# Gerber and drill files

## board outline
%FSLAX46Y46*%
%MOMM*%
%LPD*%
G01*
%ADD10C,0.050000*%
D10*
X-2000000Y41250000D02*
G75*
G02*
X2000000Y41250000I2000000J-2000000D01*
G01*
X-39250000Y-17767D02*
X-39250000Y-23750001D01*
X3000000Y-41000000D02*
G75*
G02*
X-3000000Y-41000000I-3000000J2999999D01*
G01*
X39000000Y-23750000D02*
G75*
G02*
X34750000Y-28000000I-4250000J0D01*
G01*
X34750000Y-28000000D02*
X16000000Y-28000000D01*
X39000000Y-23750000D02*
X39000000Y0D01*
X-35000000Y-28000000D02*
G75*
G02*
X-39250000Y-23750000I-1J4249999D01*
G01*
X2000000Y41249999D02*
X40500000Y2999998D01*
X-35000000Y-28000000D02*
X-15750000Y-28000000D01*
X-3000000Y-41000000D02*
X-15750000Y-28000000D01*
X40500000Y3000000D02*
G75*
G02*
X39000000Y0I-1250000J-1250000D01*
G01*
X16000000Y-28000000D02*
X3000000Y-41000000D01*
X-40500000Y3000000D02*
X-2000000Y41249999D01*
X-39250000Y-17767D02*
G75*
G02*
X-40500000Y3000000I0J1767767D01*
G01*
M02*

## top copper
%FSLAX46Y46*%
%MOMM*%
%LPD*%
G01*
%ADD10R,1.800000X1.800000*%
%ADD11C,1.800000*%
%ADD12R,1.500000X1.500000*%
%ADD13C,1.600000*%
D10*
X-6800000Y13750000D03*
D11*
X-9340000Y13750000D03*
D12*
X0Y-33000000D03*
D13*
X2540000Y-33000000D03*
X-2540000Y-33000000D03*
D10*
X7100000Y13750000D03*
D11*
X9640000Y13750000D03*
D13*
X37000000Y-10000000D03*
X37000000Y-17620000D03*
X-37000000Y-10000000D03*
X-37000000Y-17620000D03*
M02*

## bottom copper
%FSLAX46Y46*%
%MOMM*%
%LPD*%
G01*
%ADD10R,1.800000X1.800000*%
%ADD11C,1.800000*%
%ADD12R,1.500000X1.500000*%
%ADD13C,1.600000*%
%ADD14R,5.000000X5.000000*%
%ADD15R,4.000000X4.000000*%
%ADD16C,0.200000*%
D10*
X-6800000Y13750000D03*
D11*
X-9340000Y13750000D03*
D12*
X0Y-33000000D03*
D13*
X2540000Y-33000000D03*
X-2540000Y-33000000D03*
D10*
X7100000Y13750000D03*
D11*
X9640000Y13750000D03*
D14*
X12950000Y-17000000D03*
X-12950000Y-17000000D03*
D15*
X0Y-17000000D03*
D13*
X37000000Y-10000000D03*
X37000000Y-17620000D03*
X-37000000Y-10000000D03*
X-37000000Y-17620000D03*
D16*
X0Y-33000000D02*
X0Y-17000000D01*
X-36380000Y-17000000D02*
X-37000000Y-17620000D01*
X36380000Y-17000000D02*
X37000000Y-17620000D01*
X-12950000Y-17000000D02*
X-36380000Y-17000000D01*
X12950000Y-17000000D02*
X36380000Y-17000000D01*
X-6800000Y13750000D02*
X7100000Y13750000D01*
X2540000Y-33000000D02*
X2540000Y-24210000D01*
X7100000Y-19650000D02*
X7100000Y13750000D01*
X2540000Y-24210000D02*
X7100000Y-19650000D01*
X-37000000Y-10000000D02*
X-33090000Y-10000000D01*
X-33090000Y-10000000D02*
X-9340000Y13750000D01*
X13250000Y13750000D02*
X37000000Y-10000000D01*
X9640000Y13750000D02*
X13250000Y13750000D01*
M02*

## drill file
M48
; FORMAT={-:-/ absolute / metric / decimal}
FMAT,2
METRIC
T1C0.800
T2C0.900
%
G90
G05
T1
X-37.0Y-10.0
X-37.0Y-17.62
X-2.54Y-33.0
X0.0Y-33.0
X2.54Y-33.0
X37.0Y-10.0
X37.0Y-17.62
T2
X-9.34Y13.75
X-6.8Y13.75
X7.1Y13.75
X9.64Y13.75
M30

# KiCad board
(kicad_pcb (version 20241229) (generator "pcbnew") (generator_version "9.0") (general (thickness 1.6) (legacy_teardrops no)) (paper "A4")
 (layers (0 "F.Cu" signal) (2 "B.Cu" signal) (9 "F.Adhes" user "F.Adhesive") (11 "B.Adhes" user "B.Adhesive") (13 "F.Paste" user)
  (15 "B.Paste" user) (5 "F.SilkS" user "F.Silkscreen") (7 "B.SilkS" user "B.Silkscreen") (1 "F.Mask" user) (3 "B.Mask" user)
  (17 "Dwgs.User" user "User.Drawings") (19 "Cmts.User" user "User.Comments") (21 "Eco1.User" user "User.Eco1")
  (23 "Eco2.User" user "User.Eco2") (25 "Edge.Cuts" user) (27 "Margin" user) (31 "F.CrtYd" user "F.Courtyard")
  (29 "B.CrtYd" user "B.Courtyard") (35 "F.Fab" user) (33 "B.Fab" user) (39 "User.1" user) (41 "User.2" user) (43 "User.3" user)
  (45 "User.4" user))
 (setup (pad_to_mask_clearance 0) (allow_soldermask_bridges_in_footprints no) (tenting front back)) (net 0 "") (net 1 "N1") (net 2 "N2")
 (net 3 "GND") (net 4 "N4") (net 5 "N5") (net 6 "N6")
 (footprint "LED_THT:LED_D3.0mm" (layer "F.Cu") (at -6.8 -13.75 180)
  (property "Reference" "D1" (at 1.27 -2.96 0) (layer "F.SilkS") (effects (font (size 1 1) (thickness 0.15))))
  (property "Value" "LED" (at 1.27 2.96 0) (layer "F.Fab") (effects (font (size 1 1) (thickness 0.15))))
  (pad "1" thru_hole rect (at 0 0 180) (size 1.8 1.8) (drill 0.9) (layers "*.Cu" "*.Mask") (remove_unused_layers no) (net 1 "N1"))
  (pad "2" thru_hole circle (at 2.54 0 180) (size 1.8 1.8) (drill 0.9) (layers "*.Cu" "*.Mask") (remove_unused_layers no) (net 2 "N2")))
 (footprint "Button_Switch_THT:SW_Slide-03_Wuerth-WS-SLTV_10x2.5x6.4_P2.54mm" (layer "F.Cu") (at 0 33 180)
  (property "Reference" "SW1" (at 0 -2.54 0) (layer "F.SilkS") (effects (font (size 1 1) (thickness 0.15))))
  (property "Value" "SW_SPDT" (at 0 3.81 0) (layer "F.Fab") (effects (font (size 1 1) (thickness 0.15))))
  (pad "1" thru_hole rect (at 0 0 180) (size 1.5 1.5) (drill 0.8) (layers "*.Cu" "*.Mask") (remove_unused_layers no) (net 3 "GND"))
  (pad "2" thru_hole circle (at -2.54 0 180) (size 1.6 1.6) (drill 0.8) (layers "*.Cu" "*.Mask") (remove_unused_layers no) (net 1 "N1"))
  (pad "3" thru_hole circle (at 2.54 0 180) (size 1.6 1.6) (drill 0.8) (layers "*.Cu" "*.Mask") (remove_unused_layers no) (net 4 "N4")))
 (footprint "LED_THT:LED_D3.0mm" (layer "F.Cu") (at 7.1 -13.75)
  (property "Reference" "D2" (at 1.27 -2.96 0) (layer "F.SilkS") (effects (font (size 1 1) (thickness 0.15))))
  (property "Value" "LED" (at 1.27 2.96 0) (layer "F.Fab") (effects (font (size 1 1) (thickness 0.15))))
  (pad "1" thru_hole rect (at 0 0) (size 1.8 1.8) (drill 0.9) (layers "*.Cu" "*.Mask") (remove_unused_layers no) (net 1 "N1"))
  (pad "2" thru_hole circle (at 2.54 0) (size 1.8 1.8) (drill 0.9) (layers "*.Cu" "*.Mask") (remove_unused_layers no) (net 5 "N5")))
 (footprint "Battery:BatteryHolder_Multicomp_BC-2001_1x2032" (layer "B.Cu") (at 0 17 180)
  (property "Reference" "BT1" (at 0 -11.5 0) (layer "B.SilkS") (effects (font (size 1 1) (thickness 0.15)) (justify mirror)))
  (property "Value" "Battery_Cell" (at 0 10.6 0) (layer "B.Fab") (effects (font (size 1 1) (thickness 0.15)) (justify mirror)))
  (pad "1" smd rect (at -12.95 0 180) (size 5 5) (layers "B.Cu" "B.Mask" "B.Paste") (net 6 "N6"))
  (pad "1" smd rect (at 12.95 0 180) (size 5 5) (layers "B.Cu" "B.Mask" "B.Paste") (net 6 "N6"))
  (pad "2" smd rect (at 0 0 180) (size 4 4) (layers "B.Cu" "B.Mask" "B.Paste") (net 3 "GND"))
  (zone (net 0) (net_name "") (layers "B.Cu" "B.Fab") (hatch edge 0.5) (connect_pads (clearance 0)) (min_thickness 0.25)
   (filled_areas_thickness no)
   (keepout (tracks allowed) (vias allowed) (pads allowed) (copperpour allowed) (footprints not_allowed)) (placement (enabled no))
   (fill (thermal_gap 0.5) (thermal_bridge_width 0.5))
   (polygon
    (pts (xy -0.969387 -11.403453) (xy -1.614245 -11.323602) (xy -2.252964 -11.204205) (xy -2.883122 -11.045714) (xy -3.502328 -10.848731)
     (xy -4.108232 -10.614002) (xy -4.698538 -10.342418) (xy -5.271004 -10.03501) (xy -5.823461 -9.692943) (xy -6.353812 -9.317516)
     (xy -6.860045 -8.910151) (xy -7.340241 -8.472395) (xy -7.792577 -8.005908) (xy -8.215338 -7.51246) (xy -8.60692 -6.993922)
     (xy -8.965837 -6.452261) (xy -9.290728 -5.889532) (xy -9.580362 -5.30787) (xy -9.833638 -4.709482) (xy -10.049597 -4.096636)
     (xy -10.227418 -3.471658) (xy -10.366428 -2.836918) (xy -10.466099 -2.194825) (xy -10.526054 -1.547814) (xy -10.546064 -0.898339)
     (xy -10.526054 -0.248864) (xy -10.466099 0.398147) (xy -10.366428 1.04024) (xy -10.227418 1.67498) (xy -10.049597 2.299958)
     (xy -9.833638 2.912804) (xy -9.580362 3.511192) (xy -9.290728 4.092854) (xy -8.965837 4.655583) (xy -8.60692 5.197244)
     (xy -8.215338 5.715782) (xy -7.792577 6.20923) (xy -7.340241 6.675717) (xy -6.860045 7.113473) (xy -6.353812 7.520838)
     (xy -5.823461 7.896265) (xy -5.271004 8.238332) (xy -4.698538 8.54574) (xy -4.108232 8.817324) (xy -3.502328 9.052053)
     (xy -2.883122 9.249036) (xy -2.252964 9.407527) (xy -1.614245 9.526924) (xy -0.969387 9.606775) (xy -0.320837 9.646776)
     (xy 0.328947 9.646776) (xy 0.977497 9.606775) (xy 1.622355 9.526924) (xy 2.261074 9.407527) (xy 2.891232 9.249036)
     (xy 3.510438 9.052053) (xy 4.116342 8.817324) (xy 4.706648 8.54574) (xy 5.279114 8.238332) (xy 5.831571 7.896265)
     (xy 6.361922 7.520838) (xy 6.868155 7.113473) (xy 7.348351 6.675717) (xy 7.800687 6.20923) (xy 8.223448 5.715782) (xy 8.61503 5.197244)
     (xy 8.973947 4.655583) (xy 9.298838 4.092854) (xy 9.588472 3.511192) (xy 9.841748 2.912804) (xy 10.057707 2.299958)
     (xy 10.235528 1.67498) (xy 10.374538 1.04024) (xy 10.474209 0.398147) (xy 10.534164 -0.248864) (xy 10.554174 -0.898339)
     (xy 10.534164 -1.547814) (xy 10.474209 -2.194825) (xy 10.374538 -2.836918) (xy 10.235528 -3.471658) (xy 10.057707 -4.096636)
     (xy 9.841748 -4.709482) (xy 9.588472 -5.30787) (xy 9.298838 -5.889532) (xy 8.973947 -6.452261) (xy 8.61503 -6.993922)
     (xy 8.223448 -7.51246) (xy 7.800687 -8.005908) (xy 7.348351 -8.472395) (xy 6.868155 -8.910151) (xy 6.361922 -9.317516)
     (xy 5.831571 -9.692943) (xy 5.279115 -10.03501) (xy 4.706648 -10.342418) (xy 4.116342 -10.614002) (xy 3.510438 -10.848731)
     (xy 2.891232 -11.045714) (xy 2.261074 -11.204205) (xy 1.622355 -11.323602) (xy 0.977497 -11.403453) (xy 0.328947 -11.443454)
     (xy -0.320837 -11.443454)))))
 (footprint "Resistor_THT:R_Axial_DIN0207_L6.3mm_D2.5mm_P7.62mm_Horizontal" (layer "B.Cu") (at 37 10 -90)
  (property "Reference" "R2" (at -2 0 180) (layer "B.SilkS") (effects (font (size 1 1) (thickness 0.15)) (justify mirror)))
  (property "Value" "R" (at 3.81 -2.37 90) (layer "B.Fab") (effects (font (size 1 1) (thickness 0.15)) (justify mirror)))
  (pad "1" thru_hole circle (at 0 0 270) (size 1.6 1.6) (drill 0.8) (layers "*.Cu" "*.Mask") (remove_unused_layers no) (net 5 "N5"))
  (pad "2" thru_hole circle (at 7.62 0 270) (size 1.6 1.6) (drill 0.8) (layers "*.Cu" "*.Mask") (remove_unused_layers no) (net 6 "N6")))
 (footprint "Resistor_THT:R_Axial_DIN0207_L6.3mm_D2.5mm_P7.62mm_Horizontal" (layer "B.Cu") (at -37 10 -90)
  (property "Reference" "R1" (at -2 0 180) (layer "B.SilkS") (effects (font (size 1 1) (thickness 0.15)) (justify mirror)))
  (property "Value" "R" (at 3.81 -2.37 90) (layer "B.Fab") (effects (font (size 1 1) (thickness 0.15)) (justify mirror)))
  (pad "1" thru_hole circle (at 0 0 270) (size 1.6 1.6) (drill 0.8) (layers "*.Cu" "*.Mask") (remove_unused_layers no) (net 2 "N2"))
  (pad "2" thru_hole circle (at 7.62 0 270) (size 1.6 1.6) (drill 0.8) (layers "*.Cu" "*.Mask") (remove_unused_layers no) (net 6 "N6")))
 (gr_arc (start -2 -41.25) (mid 0 -42.078427) (end 2 -41.25) (stroke (width 0.05) (type default)) (layer "Edge.Cuts"))
 (gr_line (start -39.25 0.017767) (end -39.25 23.750001) (stroke (width 0.05) (type default)) (layer "Edge.Cuts"))
 (gr_arc (start 3 41) (mid 0 42.242641) (end -3 41) (stroke (width 0.05) (type default)) (layer "Edge.Cuts"))
 (gr_arc (start 39 23.75) (mid 37.755204 26.755204) (end 34.75 28) (stroke (width 0.05) (type default)) (layer "Edge.Cuts"))
 (gr_line (start 34.75 28) (end 16 28) (stroke (width 0.05) (type default)) (layer "Edge.Cuts"))
 (gr_line (start 39 23.75) (end 39 0) (stroke (width 0.05) (type default)) (layer "Edge.Cuts"))
 (gr_arc (start -35 28) (mid -38.005204 26.755204) (end -39.25 23.75) (stroke (width 0.05) (type default)) (layer "Edge.Cuts"))
 (gr_line (start 2 -41.249999) (end 40.5 -2.999998) (stroke (width 0.05) (type default)) (layer "Edge.Cuts"))
 (gr_line (start -35 28) (end -15.75 28) (stroke (width 0.05) (type default)) (layer "Edge.Cuts"))
 (gr_line (start -3 41) (end -15.75 28) (stroke (width 0.05) (type default)) (layer "Edge.Cuts"))
 (gr_arc (start 40.5 -3) (mid 40.831139 -0.959431) (end 39 0) (stroke (width 0.05) (type default)) (layer "Edge.Cuts"))
 (gr_line (start 16 28) (end 3 41) (stroke (width 0.05) (type default)) (layer "Edge.Cuts"))
 (gr_line (start -40.5 -3) (end -2 -41.249999) (stroke (width 0.05) (type default)) (layer "Edge.Cuts"))
 (gr_arc (start -39.25 0.017767) (mid -40.883204 -1.073505) (end -40.5 -3) (stroke (width 0.05) (type default)) (layer "Edge.Cuts"))
 (segment (start 0 33) (end 0 17) (width 0.2) (layer "B.Cu") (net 3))
 (segment (start -36.38 17) (end -37 17.62) (width 0.2) (layer "B.Cu") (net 6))
 (segment (start 36.38 17) (end 37 17.62) (width 0.2) (layer "B.Cu") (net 6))
 (segment (start -12.95 17) (end -36.38 17) (width 0.2) (layer "B.Cu") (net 6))
 (segment (start 12.95 17) (end 36.38 17) (width 0.2) (layer "B.Cu") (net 6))
 (segment (start -6.8 -13.75) (end 7.1 -13.75) (width 0.2) (layer "B.Cu") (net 1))
 (segment (start 2.54 33) (end 2.54 24.21) (width 0.2) (layer "B.Cu") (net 1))
 (segment (start 7.1 19.65) (end 7.1 -13.75) (width 0.2) (layer "B.Cu") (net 1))
 (segment (start 2.54 24.21) (end 7.1 19.65) (width 0.2) (layer "B.Cu") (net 1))
 (segment (start -37 10) (end -33.09 10) (width 0.2) (layer "B.Cu") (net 2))
 (segment (start -33.09 10) (end -9.34 -13.75) (width 0.2) (layer "B.Cu") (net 2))
 (segment (start 13.25 -13.75) (end 37 10) (width 0.2) (layer "B.Cu") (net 5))
 (segment (start 9.64 -13.75) (end 13.25 -13.75) (width 0.2) (layer "B.Cu") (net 5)))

